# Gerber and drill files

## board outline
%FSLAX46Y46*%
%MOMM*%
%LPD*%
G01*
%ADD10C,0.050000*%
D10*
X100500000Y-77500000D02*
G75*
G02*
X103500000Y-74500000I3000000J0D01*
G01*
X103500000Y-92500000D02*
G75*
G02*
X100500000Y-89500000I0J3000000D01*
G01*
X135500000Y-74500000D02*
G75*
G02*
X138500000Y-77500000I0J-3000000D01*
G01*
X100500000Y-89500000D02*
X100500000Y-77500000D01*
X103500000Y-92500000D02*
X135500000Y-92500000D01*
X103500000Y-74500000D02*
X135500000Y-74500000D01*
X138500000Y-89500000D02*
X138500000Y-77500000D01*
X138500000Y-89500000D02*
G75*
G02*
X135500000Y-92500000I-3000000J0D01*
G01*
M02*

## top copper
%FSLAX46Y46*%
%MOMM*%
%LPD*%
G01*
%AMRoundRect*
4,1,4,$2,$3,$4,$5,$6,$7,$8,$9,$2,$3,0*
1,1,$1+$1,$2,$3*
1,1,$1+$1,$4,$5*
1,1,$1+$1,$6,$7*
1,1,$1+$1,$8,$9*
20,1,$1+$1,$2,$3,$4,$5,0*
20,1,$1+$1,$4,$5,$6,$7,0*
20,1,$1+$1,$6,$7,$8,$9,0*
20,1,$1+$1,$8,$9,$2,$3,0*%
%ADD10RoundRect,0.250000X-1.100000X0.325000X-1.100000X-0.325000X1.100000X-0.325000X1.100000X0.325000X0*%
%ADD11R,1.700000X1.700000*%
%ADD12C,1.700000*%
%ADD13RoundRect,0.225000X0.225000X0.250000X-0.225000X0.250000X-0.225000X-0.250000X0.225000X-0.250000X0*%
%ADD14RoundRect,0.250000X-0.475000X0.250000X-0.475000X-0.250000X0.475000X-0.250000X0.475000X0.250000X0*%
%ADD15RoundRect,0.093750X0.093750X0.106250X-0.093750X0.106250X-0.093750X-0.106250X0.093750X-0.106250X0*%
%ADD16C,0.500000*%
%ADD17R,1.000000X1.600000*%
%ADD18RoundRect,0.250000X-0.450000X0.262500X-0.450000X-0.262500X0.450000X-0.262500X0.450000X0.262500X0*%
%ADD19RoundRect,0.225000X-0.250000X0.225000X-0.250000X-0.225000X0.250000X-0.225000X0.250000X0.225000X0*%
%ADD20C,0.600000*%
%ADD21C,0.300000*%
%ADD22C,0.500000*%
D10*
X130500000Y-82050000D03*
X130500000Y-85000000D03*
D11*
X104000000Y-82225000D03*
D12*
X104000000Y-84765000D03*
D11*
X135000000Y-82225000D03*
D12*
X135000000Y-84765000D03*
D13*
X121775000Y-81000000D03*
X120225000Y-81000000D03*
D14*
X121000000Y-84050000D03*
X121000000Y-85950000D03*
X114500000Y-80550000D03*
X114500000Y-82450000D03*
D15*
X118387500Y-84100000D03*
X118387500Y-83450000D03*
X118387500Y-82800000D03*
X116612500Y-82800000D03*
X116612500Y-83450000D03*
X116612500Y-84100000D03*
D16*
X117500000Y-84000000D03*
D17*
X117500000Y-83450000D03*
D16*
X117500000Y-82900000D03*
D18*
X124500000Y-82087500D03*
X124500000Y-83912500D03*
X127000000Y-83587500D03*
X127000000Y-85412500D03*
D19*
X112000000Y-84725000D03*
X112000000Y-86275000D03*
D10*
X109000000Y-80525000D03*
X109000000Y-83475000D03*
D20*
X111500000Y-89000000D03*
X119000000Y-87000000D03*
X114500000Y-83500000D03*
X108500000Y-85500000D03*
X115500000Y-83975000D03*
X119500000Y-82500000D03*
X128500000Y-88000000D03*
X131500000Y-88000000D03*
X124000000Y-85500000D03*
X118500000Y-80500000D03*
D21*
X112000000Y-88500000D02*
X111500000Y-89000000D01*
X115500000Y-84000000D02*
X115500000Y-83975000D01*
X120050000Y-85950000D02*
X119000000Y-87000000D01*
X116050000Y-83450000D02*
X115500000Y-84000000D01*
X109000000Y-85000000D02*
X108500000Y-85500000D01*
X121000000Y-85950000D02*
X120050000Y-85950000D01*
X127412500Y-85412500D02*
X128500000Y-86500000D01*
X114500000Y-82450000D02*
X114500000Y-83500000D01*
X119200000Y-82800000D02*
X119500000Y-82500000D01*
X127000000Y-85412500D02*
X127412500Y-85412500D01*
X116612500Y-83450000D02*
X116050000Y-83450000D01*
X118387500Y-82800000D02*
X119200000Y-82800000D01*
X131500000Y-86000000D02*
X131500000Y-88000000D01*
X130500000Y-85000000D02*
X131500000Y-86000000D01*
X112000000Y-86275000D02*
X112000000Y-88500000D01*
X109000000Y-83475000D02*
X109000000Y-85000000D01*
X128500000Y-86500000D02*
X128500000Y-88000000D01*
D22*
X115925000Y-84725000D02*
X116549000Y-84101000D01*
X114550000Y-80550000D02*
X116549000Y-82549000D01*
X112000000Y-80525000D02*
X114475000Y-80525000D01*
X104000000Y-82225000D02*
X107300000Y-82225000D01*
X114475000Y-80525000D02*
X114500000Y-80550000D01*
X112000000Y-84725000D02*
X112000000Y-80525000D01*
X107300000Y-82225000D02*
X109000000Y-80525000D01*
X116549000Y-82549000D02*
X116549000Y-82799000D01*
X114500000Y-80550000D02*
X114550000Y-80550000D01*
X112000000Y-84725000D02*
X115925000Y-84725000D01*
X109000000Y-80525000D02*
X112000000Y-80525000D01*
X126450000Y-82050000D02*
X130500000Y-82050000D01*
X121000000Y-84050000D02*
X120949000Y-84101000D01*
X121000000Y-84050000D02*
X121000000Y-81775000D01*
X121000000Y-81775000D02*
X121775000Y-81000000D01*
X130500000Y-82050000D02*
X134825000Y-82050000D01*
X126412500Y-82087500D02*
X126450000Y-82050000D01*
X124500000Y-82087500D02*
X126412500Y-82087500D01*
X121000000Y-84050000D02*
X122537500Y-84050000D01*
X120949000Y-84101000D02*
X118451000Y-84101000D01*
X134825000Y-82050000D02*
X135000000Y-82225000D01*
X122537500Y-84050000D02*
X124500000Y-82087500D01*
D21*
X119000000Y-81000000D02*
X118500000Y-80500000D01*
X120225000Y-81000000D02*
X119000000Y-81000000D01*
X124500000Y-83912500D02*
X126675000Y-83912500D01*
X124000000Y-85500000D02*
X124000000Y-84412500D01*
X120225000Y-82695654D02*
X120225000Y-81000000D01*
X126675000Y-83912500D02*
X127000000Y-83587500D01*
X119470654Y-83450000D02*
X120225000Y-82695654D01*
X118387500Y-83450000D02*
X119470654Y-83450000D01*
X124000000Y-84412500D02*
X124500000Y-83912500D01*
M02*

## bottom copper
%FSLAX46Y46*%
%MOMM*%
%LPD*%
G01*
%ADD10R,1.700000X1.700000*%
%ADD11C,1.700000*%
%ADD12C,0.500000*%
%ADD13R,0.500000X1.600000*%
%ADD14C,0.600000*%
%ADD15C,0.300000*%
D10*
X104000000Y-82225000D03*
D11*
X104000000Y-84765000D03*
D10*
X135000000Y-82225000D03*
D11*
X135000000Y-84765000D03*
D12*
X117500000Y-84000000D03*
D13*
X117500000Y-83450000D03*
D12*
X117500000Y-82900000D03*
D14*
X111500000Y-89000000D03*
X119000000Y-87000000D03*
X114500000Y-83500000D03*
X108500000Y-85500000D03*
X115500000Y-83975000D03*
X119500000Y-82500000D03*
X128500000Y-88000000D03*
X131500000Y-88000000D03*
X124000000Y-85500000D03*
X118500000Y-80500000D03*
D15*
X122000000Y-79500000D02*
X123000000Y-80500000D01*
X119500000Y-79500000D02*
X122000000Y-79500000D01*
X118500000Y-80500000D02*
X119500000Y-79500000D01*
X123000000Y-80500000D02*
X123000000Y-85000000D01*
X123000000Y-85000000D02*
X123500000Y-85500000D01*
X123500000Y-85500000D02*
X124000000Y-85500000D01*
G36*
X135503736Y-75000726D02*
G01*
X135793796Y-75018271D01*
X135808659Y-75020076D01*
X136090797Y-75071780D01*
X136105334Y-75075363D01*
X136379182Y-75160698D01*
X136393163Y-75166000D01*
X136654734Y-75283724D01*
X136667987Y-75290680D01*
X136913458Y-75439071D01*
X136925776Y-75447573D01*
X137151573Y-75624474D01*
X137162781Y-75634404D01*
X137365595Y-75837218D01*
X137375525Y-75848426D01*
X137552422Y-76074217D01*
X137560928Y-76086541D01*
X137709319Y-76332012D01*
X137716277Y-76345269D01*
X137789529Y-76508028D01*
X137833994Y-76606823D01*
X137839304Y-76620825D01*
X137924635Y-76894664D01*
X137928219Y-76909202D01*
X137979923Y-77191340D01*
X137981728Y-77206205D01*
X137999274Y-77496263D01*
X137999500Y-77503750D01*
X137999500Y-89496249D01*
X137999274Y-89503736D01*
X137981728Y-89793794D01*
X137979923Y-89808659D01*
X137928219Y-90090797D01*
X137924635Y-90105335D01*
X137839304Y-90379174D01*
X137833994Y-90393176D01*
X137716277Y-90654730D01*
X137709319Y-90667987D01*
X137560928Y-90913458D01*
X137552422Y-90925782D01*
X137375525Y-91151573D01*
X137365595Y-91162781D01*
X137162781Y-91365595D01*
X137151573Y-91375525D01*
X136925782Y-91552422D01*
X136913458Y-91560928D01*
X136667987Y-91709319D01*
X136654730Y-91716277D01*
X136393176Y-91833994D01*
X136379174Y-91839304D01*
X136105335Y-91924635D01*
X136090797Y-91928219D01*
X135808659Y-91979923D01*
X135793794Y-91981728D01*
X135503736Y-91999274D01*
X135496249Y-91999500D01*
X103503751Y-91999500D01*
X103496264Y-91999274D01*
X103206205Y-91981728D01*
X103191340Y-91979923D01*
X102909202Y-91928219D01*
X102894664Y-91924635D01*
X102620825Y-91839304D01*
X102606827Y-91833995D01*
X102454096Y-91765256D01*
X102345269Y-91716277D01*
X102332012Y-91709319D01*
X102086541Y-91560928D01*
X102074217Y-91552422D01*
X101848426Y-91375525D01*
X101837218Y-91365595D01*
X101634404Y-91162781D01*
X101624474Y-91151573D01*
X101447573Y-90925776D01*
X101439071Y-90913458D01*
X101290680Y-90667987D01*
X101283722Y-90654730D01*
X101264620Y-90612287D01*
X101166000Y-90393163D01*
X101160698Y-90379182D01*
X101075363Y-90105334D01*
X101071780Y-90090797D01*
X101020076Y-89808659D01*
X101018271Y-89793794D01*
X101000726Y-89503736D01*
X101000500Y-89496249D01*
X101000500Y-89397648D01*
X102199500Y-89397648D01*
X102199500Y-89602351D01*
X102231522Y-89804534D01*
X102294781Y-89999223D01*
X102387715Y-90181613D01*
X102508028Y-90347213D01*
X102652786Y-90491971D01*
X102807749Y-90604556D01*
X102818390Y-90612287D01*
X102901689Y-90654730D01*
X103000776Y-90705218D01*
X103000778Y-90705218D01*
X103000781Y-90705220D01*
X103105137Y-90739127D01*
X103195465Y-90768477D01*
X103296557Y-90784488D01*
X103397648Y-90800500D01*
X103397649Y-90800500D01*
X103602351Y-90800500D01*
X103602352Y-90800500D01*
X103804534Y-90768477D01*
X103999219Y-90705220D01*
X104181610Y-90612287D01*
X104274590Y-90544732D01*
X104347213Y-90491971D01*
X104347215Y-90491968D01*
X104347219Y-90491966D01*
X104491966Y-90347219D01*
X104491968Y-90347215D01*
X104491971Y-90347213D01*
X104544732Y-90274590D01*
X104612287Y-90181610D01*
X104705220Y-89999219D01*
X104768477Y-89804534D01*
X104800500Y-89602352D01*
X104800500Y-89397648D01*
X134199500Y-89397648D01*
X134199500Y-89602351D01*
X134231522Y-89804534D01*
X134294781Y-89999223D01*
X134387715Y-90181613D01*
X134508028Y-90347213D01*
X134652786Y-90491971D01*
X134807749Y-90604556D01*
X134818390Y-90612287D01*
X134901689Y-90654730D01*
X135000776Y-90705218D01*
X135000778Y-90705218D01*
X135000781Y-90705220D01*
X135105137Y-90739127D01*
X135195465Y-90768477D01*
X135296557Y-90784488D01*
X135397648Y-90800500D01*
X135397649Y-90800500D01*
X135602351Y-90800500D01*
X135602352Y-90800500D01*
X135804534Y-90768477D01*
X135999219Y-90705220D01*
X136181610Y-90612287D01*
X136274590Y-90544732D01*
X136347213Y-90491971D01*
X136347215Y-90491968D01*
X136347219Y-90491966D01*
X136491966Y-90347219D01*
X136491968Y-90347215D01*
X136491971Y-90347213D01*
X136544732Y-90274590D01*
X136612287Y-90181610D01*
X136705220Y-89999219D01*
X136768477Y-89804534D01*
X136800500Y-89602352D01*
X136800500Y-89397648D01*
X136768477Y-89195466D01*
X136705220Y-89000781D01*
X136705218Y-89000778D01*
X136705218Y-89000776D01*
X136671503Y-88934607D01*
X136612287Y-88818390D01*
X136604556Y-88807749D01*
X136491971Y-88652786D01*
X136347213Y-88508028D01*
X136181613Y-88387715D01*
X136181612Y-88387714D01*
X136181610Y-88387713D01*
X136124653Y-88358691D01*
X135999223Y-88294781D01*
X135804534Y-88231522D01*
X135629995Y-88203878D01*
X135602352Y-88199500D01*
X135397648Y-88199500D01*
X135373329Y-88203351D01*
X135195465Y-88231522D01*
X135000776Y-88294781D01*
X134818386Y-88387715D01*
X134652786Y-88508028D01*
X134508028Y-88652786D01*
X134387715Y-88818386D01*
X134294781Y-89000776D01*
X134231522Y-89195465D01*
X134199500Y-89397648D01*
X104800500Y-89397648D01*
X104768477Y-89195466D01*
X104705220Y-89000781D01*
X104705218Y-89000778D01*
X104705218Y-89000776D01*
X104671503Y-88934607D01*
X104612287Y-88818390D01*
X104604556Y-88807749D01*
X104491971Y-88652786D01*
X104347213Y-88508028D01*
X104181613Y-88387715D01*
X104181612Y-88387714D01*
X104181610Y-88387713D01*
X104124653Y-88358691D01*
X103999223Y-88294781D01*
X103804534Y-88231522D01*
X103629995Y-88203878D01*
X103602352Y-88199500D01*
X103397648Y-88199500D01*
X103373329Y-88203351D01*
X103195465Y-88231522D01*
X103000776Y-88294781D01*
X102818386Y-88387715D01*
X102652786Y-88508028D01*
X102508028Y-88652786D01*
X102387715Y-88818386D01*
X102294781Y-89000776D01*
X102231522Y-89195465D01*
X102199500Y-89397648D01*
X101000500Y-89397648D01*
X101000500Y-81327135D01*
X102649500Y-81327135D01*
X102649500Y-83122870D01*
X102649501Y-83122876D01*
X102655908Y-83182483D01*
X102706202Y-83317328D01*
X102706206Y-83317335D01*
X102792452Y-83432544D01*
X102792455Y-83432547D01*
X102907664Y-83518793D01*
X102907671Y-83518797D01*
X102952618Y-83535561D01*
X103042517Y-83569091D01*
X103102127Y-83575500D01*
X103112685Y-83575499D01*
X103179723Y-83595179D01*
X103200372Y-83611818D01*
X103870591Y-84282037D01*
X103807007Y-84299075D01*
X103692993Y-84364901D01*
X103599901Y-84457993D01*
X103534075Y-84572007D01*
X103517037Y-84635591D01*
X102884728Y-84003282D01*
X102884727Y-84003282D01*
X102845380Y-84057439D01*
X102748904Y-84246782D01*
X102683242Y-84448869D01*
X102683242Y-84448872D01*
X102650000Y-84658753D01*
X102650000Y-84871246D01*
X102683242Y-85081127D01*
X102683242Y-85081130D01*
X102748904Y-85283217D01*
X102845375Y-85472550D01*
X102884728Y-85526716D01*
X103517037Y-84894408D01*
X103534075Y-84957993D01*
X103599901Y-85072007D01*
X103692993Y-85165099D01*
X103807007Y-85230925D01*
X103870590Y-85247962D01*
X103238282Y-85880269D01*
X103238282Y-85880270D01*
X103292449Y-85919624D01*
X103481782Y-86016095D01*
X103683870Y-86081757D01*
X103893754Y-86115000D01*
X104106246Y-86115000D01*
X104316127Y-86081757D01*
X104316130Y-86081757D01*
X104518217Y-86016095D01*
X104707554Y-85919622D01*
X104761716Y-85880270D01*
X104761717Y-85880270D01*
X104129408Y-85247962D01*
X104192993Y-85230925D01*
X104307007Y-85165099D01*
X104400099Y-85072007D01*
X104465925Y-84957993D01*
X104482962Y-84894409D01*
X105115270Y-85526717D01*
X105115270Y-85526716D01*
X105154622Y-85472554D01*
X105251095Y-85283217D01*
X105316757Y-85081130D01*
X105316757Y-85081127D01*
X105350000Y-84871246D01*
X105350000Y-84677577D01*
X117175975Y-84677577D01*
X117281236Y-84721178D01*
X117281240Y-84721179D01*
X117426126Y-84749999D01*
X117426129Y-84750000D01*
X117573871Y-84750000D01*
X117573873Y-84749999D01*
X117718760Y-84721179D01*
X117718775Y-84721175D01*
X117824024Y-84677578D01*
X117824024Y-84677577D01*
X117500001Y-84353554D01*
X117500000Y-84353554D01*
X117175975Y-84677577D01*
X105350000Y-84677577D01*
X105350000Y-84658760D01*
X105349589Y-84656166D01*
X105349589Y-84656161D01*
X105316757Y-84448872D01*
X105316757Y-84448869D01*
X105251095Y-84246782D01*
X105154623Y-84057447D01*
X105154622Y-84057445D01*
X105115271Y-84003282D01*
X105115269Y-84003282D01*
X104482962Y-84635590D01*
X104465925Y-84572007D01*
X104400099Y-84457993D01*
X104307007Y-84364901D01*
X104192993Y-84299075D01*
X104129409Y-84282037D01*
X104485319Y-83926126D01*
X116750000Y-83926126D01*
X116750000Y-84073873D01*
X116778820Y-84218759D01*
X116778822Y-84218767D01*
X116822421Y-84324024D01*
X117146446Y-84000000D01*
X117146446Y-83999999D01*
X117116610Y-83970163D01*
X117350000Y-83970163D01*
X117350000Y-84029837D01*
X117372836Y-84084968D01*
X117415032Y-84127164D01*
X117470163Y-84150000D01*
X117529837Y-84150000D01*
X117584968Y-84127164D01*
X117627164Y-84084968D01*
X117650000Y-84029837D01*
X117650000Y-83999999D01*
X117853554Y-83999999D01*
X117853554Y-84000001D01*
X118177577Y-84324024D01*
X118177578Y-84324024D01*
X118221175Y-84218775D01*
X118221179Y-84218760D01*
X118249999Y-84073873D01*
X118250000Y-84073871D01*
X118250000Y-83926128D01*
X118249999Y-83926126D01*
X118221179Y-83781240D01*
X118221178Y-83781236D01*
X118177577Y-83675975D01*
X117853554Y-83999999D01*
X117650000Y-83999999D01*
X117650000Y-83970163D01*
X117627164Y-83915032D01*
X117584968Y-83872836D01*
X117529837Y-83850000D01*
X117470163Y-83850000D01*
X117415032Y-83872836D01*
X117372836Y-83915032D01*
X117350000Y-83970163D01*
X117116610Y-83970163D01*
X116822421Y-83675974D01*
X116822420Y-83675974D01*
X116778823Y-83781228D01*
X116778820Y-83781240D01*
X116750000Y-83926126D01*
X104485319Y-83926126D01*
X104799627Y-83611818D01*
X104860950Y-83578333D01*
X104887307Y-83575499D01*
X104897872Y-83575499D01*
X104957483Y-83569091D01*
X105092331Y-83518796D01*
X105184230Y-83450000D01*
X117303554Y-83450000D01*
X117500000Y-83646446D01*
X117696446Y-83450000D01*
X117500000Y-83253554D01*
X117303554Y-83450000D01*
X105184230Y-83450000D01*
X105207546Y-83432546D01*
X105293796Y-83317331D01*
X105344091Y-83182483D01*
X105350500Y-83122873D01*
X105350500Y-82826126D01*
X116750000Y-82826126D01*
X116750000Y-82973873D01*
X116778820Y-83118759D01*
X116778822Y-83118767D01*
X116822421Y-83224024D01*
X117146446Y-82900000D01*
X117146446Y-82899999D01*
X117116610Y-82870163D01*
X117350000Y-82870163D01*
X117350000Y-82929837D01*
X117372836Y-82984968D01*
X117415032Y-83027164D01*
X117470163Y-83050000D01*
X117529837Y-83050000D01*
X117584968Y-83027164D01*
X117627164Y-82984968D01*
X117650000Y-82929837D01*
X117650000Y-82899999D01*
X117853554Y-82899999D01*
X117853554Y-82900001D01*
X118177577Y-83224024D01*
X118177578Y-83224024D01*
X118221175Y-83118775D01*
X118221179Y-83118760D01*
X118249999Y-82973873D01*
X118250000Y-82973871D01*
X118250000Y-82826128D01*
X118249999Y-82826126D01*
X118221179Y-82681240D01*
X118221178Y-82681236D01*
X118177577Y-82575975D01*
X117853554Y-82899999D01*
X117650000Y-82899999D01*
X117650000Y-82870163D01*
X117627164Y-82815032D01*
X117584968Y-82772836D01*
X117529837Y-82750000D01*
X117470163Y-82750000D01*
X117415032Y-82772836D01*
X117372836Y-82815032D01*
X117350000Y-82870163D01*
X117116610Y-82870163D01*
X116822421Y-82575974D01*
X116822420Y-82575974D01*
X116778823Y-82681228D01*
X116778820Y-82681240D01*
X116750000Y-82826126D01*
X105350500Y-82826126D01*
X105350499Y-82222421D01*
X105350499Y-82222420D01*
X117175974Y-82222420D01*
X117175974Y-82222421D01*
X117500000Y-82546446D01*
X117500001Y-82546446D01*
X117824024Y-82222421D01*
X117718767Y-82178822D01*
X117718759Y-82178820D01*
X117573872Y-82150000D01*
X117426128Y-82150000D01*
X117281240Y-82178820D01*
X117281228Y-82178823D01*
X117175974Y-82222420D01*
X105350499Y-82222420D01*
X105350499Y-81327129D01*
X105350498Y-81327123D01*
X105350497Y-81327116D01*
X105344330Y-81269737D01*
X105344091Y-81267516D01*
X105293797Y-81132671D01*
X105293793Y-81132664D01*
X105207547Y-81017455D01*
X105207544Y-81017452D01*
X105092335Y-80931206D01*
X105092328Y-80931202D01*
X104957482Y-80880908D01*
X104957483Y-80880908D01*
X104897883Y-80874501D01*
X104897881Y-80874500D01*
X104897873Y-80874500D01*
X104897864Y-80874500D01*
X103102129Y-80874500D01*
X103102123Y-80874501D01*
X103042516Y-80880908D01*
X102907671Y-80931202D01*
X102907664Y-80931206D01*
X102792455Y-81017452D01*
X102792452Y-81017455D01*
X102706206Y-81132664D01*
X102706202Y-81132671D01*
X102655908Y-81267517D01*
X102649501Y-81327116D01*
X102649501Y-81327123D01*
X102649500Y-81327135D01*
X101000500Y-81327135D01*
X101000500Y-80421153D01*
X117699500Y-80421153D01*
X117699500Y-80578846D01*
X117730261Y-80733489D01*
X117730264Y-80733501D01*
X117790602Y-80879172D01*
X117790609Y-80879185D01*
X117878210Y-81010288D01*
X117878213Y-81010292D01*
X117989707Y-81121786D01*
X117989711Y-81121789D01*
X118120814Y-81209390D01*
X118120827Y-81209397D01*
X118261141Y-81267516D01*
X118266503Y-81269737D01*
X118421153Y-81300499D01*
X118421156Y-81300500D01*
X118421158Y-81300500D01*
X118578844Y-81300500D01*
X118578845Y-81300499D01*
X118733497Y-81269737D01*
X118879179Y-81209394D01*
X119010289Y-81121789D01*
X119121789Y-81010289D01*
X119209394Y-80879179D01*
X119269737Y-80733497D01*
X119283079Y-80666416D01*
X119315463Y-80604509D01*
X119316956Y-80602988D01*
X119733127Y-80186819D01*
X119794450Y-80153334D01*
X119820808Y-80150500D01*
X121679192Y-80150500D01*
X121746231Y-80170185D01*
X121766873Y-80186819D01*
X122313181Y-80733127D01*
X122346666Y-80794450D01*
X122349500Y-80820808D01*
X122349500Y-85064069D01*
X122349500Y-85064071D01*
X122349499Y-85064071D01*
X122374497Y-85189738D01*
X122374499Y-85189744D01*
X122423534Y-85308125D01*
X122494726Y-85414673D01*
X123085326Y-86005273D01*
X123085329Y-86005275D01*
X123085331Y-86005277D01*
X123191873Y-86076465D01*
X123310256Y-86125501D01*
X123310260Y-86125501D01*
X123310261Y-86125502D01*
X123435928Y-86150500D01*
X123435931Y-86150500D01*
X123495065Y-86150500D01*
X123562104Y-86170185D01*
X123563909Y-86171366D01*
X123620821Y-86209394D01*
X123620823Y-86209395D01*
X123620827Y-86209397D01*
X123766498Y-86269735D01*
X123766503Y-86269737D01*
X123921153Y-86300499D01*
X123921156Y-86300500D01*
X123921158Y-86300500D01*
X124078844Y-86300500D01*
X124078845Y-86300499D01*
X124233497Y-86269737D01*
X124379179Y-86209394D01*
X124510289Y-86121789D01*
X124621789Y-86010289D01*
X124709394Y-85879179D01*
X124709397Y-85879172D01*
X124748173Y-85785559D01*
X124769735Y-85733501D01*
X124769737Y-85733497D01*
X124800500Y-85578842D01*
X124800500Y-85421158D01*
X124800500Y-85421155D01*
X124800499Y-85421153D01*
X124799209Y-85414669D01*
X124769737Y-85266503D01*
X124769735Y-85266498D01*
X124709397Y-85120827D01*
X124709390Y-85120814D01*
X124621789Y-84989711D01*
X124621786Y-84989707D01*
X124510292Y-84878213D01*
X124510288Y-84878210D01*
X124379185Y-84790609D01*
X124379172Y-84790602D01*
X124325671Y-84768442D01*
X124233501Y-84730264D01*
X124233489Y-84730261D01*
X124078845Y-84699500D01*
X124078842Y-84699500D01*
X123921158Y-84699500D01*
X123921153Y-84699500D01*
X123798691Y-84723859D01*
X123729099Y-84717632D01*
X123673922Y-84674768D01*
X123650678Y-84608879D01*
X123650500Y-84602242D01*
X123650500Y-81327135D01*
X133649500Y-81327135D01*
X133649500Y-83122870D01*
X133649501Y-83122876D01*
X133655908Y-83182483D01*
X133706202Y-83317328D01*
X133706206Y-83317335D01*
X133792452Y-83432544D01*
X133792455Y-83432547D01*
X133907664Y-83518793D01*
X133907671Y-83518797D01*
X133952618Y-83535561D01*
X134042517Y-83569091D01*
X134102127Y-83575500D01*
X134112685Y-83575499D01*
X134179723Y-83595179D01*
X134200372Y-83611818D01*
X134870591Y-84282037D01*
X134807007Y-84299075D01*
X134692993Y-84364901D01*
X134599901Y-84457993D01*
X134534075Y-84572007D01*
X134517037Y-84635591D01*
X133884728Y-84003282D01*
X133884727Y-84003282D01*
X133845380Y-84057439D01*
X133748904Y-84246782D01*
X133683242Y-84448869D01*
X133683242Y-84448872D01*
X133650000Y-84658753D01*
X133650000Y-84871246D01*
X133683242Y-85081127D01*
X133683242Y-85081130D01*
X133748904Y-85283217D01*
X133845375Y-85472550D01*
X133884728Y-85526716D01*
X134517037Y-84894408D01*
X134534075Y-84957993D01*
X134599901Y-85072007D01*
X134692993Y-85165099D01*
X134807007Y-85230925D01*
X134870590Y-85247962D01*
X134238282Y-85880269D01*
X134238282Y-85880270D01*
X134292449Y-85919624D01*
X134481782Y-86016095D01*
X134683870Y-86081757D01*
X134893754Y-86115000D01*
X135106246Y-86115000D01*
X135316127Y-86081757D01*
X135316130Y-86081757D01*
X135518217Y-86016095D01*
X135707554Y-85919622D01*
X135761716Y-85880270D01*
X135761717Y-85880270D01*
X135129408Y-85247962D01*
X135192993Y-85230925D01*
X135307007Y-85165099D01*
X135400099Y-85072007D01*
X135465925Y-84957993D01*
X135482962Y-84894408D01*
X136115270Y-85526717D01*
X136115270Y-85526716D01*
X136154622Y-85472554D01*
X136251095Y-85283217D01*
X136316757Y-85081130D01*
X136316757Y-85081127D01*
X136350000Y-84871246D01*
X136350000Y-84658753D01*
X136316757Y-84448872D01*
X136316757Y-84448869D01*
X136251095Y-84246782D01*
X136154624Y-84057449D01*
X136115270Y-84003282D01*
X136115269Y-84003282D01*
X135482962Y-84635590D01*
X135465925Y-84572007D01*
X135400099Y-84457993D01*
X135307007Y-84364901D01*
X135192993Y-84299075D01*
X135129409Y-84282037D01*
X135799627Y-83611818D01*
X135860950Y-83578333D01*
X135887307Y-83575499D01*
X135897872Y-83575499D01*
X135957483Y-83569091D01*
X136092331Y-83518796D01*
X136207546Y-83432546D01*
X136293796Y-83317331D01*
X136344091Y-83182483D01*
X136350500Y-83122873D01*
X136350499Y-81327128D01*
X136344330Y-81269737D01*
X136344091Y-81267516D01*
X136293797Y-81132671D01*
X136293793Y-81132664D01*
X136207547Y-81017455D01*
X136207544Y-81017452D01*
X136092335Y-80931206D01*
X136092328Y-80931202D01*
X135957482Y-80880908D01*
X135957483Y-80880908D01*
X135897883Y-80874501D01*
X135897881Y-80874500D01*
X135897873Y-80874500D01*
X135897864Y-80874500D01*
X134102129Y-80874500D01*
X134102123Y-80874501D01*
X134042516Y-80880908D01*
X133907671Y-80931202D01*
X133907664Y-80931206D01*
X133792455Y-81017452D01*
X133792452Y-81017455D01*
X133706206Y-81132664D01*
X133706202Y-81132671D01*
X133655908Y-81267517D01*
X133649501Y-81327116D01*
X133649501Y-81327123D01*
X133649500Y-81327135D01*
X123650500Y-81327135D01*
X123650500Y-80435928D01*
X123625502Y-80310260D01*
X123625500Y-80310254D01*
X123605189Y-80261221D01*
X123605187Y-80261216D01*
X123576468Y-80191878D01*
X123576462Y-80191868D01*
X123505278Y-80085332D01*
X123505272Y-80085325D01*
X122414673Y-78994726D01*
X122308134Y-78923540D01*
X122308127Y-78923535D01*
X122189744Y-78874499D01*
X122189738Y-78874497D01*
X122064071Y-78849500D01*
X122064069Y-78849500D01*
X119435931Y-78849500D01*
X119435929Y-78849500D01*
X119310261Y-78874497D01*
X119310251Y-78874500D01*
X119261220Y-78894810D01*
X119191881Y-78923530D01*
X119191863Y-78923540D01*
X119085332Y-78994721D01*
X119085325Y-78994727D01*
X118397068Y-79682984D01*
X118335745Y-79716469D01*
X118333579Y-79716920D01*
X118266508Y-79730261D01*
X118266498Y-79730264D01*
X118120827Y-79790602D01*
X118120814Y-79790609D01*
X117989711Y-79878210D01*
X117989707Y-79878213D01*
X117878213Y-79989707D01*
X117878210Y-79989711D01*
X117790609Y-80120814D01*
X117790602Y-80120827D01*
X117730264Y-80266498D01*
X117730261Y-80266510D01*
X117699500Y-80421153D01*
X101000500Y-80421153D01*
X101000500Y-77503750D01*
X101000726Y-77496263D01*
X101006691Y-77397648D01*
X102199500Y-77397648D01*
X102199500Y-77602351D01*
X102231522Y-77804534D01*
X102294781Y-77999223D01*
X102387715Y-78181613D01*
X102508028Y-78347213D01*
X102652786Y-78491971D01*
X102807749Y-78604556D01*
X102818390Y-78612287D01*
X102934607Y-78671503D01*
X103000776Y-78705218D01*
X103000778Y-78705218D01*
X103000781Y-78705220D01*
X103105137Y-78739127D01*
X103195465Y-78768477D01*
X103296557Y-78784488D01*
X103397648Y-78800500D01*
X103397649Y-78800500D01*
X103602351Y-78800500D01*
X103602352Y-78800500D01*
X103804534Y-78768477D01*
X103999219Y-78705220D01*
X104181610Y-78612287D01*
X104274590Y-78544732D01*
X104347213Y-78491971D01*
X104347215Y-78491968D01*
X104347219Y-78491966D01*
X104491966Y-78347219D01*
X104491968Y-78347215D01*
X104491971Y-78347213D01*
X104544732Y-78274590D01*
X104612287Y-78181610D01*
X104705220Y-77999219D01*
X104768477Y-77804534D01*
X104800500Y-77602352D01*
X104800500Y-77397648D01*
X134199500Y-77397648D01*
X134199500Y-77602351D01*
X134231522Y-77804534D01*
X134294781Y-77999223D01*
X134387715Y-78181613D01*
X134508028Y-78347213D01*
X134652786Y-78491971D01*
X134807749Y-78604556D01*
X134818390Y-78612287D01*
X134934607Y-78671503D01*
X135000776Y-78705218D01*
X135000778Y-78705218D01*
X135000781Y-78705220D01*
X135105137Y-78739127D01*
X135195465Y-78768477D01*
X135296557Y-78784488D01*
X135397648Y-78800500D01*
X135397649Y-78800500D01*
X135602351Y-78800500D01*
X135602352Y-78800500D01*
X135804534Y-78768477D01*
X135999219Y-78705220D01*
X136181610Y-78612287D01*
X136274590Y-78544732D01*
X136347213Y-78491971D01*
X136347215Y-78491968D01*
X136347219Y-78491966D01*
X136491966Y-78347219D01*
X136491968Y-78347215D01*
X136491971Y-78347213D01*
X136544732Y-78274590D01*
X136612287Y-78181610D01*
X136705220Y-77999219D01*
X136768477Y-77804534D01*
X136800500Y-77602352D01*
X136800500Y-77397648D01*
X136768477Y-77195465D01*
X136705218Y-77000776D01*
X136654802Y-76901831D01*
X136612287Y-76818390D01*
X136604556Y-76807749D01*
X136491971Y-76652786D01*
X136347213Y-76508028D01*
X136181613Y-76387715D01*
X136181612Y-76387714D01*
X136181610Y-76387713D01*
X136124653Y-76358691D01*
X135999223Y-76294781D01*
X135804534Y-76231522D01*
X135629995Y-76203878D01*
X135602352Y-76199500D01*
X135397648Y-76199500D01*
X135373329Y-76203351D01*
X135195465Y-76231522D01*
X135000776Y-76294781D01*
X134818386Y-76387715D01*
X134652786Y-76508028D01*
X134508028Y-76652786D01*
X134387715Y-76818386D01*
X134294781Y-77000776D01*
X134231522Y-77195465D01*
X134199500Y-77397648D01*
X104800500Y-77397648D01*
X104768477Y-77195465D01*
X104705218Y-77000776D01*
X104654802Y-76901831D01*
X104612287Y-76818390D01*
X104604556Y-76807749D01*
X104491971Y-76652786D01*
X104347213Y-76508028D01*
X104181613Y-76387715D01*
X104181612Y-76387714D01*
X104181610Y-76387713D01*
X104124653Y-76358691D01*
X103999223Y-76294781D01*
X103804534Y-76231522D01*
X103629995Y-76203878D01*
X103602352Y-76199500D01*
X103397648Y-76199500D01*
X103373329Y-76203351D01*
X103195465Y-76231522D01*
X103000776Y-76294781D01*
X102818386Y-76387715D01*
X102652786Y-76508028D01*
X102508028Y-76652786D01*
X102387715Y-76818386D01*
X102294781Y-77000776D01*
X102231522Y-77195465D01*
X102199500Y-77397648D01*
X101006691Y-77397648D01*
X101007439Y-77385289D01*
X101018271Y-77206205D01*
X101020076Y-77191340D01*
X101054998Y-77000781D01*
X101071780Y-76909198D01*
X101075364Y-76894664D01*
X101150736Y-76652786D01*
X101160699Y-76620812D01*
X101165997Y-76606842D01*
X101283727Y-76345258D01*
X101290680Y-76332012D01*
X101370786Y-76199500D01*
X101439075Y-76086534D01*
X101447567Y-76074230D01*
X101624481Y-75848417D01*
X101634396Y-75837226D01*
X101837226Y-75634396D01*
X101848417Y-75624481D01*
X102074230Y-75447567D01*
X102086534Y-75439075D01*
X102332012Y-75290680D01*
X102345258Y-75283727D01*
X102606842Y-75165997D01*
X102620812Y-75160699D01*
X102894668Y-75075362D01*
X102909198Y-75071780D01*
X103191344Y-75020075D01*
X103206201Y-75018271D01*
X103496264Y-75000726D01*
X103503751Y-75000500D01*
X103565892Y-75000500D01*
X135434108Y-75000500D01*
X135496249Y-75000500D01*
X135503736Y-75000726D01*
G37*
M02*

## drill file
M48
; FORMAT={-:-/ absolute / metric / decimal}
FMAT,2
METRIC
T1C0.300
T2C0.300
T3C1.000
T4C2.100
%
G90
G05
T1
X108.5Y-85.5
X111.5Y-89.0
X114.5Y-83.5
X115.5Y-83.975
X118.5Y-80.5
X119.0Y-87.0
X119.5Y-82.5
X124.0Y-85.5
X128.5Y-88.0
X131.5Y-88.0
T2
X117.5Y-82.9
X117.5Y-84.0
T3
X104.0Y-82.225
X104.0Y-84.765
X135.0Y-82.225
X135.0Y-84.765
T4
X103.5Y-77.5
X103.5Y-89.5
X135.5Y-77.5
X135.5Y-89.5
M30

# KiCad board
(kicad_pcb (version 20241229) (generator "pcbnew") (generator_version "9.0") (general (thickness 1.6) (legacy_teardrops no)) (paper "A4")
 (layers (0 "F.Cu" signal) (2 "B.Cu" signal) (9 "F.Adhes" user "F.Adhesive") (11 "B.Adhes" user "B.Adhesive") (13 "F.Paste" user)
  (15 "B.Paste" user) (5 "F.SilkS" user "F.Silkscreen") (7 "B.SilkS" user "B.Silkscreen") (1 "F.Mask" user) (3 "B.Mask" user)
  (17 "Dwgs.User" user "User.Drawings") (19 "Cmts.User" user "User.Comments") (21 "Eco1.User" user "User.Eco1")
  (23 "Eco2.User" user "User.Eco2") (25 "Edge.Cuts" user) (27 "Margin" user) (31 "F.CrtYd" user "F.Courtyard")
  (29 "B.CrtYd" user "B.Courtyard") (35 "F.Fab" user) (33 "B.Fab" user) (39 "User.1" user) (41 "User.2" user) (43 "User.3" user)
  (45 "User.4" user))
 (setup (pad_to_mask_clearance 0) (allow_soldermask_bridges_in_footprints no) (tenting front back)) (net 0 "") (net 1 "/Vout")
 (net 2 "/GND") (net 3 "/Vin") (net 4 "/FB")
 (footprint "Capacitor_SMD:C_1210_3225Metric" (layer "F.Cu") (at 130.5 83.525 -90)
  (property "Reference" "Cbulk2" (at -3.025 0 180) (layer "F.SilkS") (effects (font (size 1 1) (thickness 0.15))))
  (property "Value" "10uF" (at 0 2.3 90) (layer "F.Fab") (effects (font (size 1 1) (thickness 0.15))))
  (pad "1" smd roundrect (at -1.475 0 270) (size 1.15 2.7) (layers "F.Cu" "F.Mask" "F.Paste") (roundrect_rratio 0.217391) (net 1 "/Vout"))
  (pad "2" smd roundrect (at 1.475 0 270) (size 1.15 2.7) (layers "F.Cu" "F.Mask" "F.Paste") (roundrect_rratio 0.217391) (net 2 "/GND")))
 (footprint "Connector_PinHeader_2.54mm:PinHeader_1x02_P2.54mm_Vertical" (layer "F.Cu") (at 104 82.225)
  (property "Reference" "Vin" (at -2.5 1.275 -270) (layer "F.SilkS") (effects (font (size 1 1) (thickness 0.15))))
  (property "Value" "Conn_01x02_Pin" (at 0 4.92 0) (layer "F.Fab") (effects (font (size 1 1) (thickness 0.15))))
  (pad "1" thru_hole rect (at 0 0) (size 1.7 1.7) (drill 1) (layers "*.Cu" "*.Mask") (remove_unused_layers no) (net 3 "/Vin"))
  (pad "2" thru_hole circle (at 0 2.54) (size 1.7 1.7) (drill 1) (layers "*.Cu" "*.Mask") (remove_unused_layers no) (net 2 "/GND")))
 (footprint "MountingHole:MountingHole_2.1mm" (layer "F.Cu") (at 103.5 89.5)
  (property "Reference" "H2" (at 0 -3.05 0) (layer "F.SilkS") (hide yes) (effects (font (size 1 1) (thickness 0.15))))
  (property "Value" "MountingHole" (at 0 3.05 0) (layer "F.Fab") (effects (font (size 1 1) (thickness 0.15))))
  (pad "" np_thru_hole circle (at 0 0) (size 2.1 2.1) (drill 2.1) (layers "*.Cu" "*.Mask")))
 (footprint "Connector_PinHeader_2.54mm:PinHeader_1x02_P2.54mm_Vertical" (layer "F.Cu") (at 135 82.225)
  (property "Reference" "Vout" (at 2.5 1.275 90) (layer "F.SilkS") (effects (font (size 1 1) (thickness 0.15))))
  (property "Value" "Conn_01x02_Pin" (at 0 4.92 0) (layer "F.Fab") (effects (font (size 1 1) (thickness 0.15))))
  (pad "1" thru_hole rect (at 0 0) (size 1.7 1.7) (drill 1) (layers "*.Cu" "*.Mask") (remove_unused_layers no) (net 1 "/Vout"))
  (pad "2" thru_hole circle (at 0 2.54) (size 1.7 1.7) (drill 1) (layers "*.Cu" "*.Mask") (remove_unused_layers no) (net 2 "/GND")))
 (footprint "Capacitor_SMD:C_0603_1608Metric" (layer "F.Cu") (at 121 81 180)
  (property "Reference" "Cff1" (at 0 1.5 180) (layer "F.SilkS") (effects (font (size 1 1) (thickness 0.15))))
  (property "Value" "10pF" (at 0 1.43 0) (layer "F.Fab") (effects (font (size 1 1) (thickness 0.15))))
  (pad "1" smd roundrect (at -0.775 0 180) (size 0.9 0.95) (layers "F.Cu" "F.Mask" "F.Paste") (roundrect_rratio 0.25) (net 1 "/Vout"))
  (pad "2" smd roundrect (at 0.775 0 180) (size 0.9 0.95) (layers "F.Cu" "F.Mask" "F.Paste") (roundrect_rratio 0.25) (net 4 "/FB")))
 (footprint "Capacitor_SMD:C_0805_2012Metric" (layer "F.Cu") (at 121 85 -90)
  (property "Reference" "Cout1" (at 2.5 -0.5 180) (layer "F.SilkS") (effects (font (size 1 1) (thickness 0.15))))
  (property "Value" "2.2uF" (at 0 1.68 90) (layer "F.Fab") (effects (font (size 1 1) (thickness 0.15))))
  (pad "1" smd roundrect (at -0.95 0 270) (size 1 1.45) (layers "F.Cu" "F.Mask" "F.Paste") (roundrect_rratio 0.25) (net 1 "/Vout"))
  (pad "2" smd roundrect (at 0.95 0 270) (size 1 1.45) (layers "F.Cu" "F.Mask" "F.Paste") (roundrect_rratio 0.25) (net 2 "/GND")))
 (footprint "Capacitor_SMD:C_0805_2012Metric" (layer "F.Cu") (at 114.5 81.5 -90)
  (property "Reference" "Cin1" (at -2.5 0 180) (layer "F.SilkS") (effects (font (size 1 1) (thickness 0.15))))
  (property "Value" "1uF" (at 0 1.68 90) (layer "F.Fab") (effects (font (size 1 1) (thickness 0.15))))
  (pad "1" smd roundrect (at -0.95 0 270) (size 1 1.45) (layers "F.Cu" "F.Mask" "F.Paste") (roundrect_rratio 0.25) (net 3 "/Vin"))
  (pad "2" smd roundrect (at 0.95 0 270) (size 1 1.45) (layers "F.Cu" "F.Mask" "F.Paste") (roundrect_rratio 0.25) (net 2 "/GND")))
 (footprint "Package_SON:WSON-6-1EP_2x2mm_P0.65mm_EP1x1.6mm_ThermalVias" (layer "F.Cu") (at 117.5 83.45 180)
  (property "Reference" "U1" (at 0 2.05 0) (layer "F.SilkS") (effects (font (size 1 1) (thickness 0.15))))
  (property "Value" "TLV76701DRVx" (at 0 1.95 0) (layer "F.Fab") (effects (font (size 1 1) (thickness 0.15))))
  (pad "" smd roundrect (at 0 -0.4 180) (size 0.87 0.69) (layers "F.Paste") (roundrect_rratio 0.25))
  (pad "" smd roundrect (at 0 0.4 180) (size 0.87 0.69) (layers "F.Paste") (roundrect_rratio 0.25))
  (pad "1" smd roundrect (at -0.8875 -0.65 180) (size 0.375 0.4) (layers "F.Cu" "F.Mask" "F.Paste") (roundrect_rratio 0.25) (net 1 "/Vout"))
  (pad "2" smd roundrect (at -0.8875 0 180) (size 0.375 0.4) (layers "F.Cu" "F.Mask" "F.Paste") (roundrect_rratio 0.25) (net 4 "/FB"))
  (pad "3" smd roundrect (at -0.8875 0.65 180) (size 0.375 0.4) (layers "F.Cu" "F.Mask" "F.Paste") (roundrect_rratio 0.25) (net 2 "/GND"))
  (pad "4" smd roundrect (at 0.8875 0.65 180) (size 0.375 0.4) (layers "F.Cu" "F.Mask" "F.Paste") (roundrect_rratio 0.25) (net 3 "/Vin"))
  (pad "5" smd roundrect (at 0.8875 0 180) (size 0.375 0.4) (layers "F.Cu" "F.Mask" "F.Paste") (roundrect_rratio 0.25) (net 2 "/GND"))
  (pad "6" smd roundrect (at 0.8875 -0.65 180) (size 0.375 0.4) (layers "F.Cu" "F.Mask" "F.Paste") (roundrect_rratio 0.25) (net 3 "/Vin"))
  (pad "7" thru_hole circle (at 0 -0.55 180) (size 0.5 0.5) (drill 0.3) (layers "*.Cu") (remove_unused_layers no) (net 2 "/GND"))
  (pad "7" smd rect (at 0 0 180) (size 0.5 1.6) (layers "B.Cu") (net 2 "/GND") (zone_connect 2))
  (pad "7" smd rect (at 0 0 180) (size 1 1.6) (layers "F.Cu" "F.Mask") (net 2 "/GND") (zone_connect 2))
  (pad "7" thru_hole circle (at 0 0.55 180) (size 0.5 0.5) (drill 0.3) (layers "*.Cu") (remove_unused_layers no) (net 2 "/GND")))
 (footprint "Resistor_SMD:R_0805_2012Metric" (layer "F.Cu") (at 124.5 83 -90)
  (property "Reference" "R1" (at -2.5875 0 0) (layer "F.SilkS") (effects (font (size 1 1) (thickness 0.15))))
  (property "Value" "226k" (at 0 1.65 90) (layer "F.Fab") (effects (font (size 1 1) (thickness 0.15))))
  (pad "1" smd roundrect (at -0.9125 0 270) (size 1.025 1.4) (layers "F.Cu" "F.Mask" "F.Paste") (roundrect_rratio 0.243902) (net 1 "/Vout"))
  (pad "2" smd roundrect (at 0.9125 0 270) (size 1.025 1.4) (layers "F.Cu" "F.Mask" "F.Paste") (roundrect_rratio 0.243902) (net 4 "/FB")))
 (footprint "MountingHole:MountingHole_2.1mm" (layer "F.Cu") (at 135.5 77.5)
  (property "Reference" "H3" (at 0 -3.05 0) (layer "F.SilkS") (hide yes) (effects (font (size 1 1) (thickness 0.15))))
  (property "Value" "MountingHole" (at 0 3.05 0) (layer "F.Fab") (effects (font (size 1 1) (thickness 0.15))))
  (pad "" np_thru_hole circle (at 0 0) (size 2.1 2.1) (drill 2.1) (layers "*.Cu" "*.Mask")))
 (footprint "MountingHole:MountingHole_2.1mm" (layer "F.Cu") (at 103.5 77.5)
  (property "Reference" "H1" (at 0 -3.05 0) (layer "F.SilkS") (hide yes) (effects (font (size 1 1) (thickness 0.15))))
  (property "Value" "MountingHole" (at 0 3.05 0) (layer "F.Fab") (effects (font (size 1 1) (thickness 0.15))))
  (pad "" np_thru_hole circle (at 0 0) (size 2.1 2.1) (drill 2.1) (layers "*.Cu" "*.Mask")))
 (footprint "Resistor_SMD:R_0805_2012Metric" (layer "F.Cu") (at 127 84.5 -90)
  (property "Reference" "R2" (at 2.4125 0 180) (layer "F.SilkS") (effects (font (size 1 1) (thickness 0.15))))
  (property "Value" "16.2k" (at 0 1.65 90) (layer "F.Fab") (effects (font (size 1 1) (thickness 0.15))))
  (pad "1" smd roundrect (at -0.9125 0 270) (size 1.025 1.4) (layers "F.Cu" "F.Mask" "F.Paste") (roundrect_rratio 0.243902) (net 4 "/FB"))
  (pad "2" smd roundrect (at 0.9125 0 270) (size 1.025 1.4) (layers "F.Cu" "F.Mask" "F.Paste") (roundrect_rratio 0.243902) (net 2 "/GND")))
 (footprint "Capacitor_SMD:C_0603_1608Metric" (layer "F.Cu") (at 112 85.5 -90)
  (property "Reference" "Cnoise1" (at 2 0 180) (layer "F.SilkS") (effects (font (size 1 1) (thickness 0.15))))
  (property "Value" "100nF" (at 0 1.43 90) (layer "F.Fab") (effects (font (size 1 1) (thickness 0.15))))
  (pad "1" smd roundrect (at -0.775 0 270) (size 0.9 0.95) (layers "F.Cu" "F.Mask" "F.Paste") (roundrect_rratio 0.25) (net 3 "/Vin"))
  (pad "2" smd roundrect (at 0.775 0 270) (size 0.9 0.95) (layers "F.Cu" "F.Mask" "F.Paste") (roundrect_rratio 0.25) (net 2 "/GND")))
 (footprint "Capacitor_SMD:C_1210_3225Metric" (layer "F.Cu") (at 109 82 -90)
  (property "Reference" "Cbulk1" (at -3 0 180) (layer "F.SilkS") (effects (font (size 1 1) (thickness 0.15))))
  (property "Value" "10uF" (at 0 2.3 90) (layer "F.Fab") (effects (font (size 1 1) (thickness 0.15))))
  (pad "1" smd roundrect (at -1.475 0 270) (size 1.15 2.7) (layers "F.Cu" "F.Mask" "F.Paste") (roundrect_rratio 0.217391) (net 3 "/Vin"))
  (pad "2" smd roundrect (at 1.475 0 270) (size 1.15 2.7) (layers "F.Cu" "F.Mask" "F.Paste") (roundrect_rratio 0.217391) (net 2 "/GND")))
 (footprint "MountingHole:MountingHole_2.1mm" (layer "F.Cu") (at 135.5 89.5)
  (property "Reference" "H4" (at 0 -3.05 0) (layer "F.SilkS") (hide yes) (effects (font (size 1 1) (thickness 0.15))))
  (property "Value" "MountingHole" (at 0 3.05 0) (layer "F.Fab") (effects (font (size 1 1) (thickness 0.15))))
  (pad "" np_thru_hole circle (at 0 0) (size 2.1 2.1) (drill 2.1) (layers "*.Cu" "*.Mask")))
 (gr_arc (start 100.5 77.5) (mid 101.37868 75.37868) (end 103.5 74.5) (stroke (width 0.05) (type default)) (layer "Edge.Cuts"))
 (gr_arc (start 103.5 92.5) (mid 101.37868 91.62132) (end 100.5 89.5) (stroke (width 0.05) (type default)) (layer "Edge.Cuts"))
 (gr_arc (start 135.5 74.5) (mid 137.62132 75.37868) (end 138.5 77.5) (stroke (width 0.05) (type default)) (layer "Edge.Cuts"))
 (gr_line (start 100.5 89.5) (end 100.5 77.5) (stroke (width 0.05) (type default)) (layer "Edge.Cuts"))
 (gr_line (start 103.5 92.5) (end 135.5 92.5) (stroke (width 0.05) (type default)) (layer "Edge.Cuts"))
 (gr_line (start 103.5 74.5) (end 135.5 74.5) (stroke (width 0.05) (type default)) (layer "Edge.Cuts"))
 (gr_line (start 138.5 89.5) (end 138.5 77.5) (stroke (width 0.05) (type default)) (layer "Edge.Cuts"))
 (gr_arc (start 138.5 89.5) (mid 137.62132 91.62132) (end 135.5 92.5) (stroke (width 0.05) (type default)) (layer "Edge.Cuts"))
 (segment (start 112 88.5) (end 111.5 89) (width 0.3) (layer "F.Cu") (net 2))
 (segment (start 115.5 84) (end 115.5 83.975) (width 0.3) (layer "F.Cu") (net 2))
 (segment (start 120.05 85.95) (end 119 87) (width 0.3) (layer "F.Cu") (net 2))
 (segment (start 116.05 83.45) (end 115.5 84) (width 0.3) (layer "F.Cu") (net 2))
 (segment (start 109 85) (end 108.5 85.5) (width 0.3) (layer "F.Cu") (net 2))
 (segment (start 121 85.95) (end 120.05 85.95) (width 0.3) (layer "F.Cu") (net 2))
 (segment (start 127.4125 85.4125) (end 128.5 86.5) (width 0.3) (layer "F.Cu") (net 2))
 (segment (start 114.5 82.45) (end 114.5 83.5) (width 0.3) (layer "F.Cu") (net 2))
 (segment (start 119.2 82.8) (end 119.5 82.5) (width 0.3) (layer "F.Cu") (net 2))
 (segment (start 127 85.4125) (end 127.4125 85.4125) (width 0.3) (layer "F.Cu") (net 2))
 (segment (start 116.6125 83.45) (end 116.05 83.45) (width 0.3) (layer "F.Cu") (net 2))
 (segment (start 118.3875 82.8) (end 119.2 82.8) (width 0.3) (layer "F.Cu") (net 2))
 (segment (start 131.5 86) (end 131.5 88) (width 0.3) (layer "F.Cu") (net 2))
 (segment (start 130.5 85) (end 131.5 86) (width 0.3) (layer "F.Cu") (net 2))
 (segment (start 112 86.275) (end 112 88.5) (width 0.3) (layer "F.Cu") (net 2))
 (segment (start 109 83.475) (end 109 85) (width 0.3) (layer "F.Cu") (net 2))
 (segment (start 128.5 86.5) (end 128.5 88) (width 0.3) (layer "F.Cu") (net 2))
 (via (at 111.5 89) (size 0.6) (drill 0.3) (layers "F.Cu" "B.Cu") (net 2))
 (via (at 119 87) (size 0.6) (drill 0.3) (layers "F.Cu" "B.Cu") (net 2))
 (via (at 114.5 83.5) (size 0.6) (drill 0.3) (layers "F.Cu" "B.Cu") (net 2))
 (via (at 108.5 85.5) (size 0.6) (drill 0.3) (layers "F.Cu" "B.Cu") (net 2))
 (via (at 115.5 83.975) (size 0.6) (drill 0.3) (layers "F.Cu" "B.Cu") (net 2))
 (via (at 119.5 82.5) (size 0.6) (drill 0.3) (layers "F.Cu" "B.Cu") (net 2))
 (via (at 128.5 88) (size 0.6) (drill 0.3) (layers "F.Cu" "B.Cu") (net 2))
 (via (at 131.5 88) (size 0.6) (drill 0.3) (layers "F.Cu" "B.Cu") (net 2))
 (segment (start 115.925 84.725) (end 116.549 84.101) (width 0.5) (layer "F.Cu") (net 3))
 (segment (start 114.55 80.55) (end 116.549 82.549) (width 0.5) (layer "F.Cu") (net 3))
 (segment (start 112 80.525) (end 114.475 80.525) (width 0.5) (layer "F.Cu") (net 3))
 (segment (start 104 82.225) (end 107.3 82.225) (width 0.5) (layer "F.Cu") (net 3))
 (segment (start 114.475 80.525) (end 114.5 80.55) (width 0.5) (layer "F.Cu") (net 3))
 (segment (start 112 84.725) (end 112 80.525) (width 0.5) (layer "F.Cu") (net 3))
 (segment (start 107.3 82.225) (end 109 80.525) (width 0.5) (layer "F.Cu") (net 3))
 (segment (start 116.549 82.549) (end 116.549 82.799) (width 0.5) (layer "F.Cu") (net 3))
 (segment (start 114.5 80.55) (end 114.55 80.55) (width 0.5) (layer "F.Cu") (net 3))
 (segment (start 112 84.725) (end 115.925 84.725) (width 0.5) (layer "F.Cu") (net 3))
 (segment (start 109 80.525) (end 112 80.525) (width 0.5) (layer "F.Cu") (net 3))
 (segment (start 126.45 82.05) (end 130.5 82.05) (width 0.5) (layer "F.Cu") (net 1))
 (segment (start 121 84.05) (end 120.949 84.101) (width 0.5) (layer "F.Cu") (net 1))
 (segment (start 121 84.05) (end 121 81.775) (width 0.5) (layer "F.Cu") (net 1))
 (segment (start 121 81.775) (end 121.775 81) (width 0.5) (layer "F.Cu") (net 1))
 (segment (start 130.5 82.05) (end 134.825 82.05) (width 0.5) (layer "F.Cu") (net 1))
 (segment (start 126.4125 82.0875) (end 126.45 82.05) (width 0.5) (layer "F.Cu") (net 1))
 (segment (start 124.5 82.0875) (end 126.4125 82.0875) (width 0.5) (layer "F.Cu") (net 1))
 (segment (start 121 84.05) (end 122.5375 84.05) (width 0.5) (layer "F.Cu") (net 1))
 (segment (start 120.949 84.101) (end 118.451 84.101) (width 0.5) (layer "F.Cu") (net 1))
 (segment (start 134.825 82.05) (end 135 82.225) (width 0.5) (layer "F.Cu") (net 1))
 (segment (start 122.5375 84.05) (end 124.5 82.0875) (width 0.5) (layer "F.Cu") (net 1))
 (segment (start 119 81) (end 118.5 80.5) (width 0.3) (layer "F.Cu") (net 4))
 (segment (start 120.225 81) (end 119 81) (width 0.3) (layer "F.Cu") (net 4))
 (segment (start 124.5 83.9125) (end 126.675 83.9125) (width 0.3) (layer "F.Cu") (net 4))
 (segment (start 124 85.5) (end 124 84.4125) (width 0.3) (layer "F.Cu") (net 4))
 (segment (start 120.225 82.695654) (end 120.225 81) (width 0.3) (layer "F.Cu") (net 4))
 (segment (start 126.675 83.9125) (end 127 83.5875) (width 0.3) (layer "F.Cu") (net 4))
 (segment (start 119.470654 83.45) (end 120.225 82.695654) (width 0.3) (layer "F.Cu") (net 4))
 (segment (start 118.3875 83.45) (end 119.470654 83.45) (width 0.3) (layer "F.Cu") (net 4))
 (segment (start 124 84.4125) (end 124.5 83.9125) (width 0.3) (layer "F.Cu") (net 4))
 (via (at 124 85.5) (size 0.6) (drill 0.3) (layers "F.Cu" "B.Cu") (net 4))
 (via (at 118.5 80.5) (size 0.6) (drill 0.3) (layers "F.Cu" "B.Cu") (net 4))
 (segment (start 122 79.5) (end 123 80.5) (width 0.3) (layer "B.Cu") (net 4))
 (segment (start 119.5 79.5) (end 122 79.5) (width 0.3) (layer "B.Cu") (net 4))
 (segment (start 118.5 80.5) (end 119.5 79.5) (width 0.3) (layer "B.Cu") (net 4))
 (segment (start 123 80.5) (end 123 85) (width 0.3) (layer "B.Cu") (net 4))
 (segment (start 123 85) (end 123.5 85.5) (width 0.3) (layer "B.Cu") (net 4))
 (segment (start 123.5 85.5) (end 124 85.5) (width 0.3) (layer "B.Cu") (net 4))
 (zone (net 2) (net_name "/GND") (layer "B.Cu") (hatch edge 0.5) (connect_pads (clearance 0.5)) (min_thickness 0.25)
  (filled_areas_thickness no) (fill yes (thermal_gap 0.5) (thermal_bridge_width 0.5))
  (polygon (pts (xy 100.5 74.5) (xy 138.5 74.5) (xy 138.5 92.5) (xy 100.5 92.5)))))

